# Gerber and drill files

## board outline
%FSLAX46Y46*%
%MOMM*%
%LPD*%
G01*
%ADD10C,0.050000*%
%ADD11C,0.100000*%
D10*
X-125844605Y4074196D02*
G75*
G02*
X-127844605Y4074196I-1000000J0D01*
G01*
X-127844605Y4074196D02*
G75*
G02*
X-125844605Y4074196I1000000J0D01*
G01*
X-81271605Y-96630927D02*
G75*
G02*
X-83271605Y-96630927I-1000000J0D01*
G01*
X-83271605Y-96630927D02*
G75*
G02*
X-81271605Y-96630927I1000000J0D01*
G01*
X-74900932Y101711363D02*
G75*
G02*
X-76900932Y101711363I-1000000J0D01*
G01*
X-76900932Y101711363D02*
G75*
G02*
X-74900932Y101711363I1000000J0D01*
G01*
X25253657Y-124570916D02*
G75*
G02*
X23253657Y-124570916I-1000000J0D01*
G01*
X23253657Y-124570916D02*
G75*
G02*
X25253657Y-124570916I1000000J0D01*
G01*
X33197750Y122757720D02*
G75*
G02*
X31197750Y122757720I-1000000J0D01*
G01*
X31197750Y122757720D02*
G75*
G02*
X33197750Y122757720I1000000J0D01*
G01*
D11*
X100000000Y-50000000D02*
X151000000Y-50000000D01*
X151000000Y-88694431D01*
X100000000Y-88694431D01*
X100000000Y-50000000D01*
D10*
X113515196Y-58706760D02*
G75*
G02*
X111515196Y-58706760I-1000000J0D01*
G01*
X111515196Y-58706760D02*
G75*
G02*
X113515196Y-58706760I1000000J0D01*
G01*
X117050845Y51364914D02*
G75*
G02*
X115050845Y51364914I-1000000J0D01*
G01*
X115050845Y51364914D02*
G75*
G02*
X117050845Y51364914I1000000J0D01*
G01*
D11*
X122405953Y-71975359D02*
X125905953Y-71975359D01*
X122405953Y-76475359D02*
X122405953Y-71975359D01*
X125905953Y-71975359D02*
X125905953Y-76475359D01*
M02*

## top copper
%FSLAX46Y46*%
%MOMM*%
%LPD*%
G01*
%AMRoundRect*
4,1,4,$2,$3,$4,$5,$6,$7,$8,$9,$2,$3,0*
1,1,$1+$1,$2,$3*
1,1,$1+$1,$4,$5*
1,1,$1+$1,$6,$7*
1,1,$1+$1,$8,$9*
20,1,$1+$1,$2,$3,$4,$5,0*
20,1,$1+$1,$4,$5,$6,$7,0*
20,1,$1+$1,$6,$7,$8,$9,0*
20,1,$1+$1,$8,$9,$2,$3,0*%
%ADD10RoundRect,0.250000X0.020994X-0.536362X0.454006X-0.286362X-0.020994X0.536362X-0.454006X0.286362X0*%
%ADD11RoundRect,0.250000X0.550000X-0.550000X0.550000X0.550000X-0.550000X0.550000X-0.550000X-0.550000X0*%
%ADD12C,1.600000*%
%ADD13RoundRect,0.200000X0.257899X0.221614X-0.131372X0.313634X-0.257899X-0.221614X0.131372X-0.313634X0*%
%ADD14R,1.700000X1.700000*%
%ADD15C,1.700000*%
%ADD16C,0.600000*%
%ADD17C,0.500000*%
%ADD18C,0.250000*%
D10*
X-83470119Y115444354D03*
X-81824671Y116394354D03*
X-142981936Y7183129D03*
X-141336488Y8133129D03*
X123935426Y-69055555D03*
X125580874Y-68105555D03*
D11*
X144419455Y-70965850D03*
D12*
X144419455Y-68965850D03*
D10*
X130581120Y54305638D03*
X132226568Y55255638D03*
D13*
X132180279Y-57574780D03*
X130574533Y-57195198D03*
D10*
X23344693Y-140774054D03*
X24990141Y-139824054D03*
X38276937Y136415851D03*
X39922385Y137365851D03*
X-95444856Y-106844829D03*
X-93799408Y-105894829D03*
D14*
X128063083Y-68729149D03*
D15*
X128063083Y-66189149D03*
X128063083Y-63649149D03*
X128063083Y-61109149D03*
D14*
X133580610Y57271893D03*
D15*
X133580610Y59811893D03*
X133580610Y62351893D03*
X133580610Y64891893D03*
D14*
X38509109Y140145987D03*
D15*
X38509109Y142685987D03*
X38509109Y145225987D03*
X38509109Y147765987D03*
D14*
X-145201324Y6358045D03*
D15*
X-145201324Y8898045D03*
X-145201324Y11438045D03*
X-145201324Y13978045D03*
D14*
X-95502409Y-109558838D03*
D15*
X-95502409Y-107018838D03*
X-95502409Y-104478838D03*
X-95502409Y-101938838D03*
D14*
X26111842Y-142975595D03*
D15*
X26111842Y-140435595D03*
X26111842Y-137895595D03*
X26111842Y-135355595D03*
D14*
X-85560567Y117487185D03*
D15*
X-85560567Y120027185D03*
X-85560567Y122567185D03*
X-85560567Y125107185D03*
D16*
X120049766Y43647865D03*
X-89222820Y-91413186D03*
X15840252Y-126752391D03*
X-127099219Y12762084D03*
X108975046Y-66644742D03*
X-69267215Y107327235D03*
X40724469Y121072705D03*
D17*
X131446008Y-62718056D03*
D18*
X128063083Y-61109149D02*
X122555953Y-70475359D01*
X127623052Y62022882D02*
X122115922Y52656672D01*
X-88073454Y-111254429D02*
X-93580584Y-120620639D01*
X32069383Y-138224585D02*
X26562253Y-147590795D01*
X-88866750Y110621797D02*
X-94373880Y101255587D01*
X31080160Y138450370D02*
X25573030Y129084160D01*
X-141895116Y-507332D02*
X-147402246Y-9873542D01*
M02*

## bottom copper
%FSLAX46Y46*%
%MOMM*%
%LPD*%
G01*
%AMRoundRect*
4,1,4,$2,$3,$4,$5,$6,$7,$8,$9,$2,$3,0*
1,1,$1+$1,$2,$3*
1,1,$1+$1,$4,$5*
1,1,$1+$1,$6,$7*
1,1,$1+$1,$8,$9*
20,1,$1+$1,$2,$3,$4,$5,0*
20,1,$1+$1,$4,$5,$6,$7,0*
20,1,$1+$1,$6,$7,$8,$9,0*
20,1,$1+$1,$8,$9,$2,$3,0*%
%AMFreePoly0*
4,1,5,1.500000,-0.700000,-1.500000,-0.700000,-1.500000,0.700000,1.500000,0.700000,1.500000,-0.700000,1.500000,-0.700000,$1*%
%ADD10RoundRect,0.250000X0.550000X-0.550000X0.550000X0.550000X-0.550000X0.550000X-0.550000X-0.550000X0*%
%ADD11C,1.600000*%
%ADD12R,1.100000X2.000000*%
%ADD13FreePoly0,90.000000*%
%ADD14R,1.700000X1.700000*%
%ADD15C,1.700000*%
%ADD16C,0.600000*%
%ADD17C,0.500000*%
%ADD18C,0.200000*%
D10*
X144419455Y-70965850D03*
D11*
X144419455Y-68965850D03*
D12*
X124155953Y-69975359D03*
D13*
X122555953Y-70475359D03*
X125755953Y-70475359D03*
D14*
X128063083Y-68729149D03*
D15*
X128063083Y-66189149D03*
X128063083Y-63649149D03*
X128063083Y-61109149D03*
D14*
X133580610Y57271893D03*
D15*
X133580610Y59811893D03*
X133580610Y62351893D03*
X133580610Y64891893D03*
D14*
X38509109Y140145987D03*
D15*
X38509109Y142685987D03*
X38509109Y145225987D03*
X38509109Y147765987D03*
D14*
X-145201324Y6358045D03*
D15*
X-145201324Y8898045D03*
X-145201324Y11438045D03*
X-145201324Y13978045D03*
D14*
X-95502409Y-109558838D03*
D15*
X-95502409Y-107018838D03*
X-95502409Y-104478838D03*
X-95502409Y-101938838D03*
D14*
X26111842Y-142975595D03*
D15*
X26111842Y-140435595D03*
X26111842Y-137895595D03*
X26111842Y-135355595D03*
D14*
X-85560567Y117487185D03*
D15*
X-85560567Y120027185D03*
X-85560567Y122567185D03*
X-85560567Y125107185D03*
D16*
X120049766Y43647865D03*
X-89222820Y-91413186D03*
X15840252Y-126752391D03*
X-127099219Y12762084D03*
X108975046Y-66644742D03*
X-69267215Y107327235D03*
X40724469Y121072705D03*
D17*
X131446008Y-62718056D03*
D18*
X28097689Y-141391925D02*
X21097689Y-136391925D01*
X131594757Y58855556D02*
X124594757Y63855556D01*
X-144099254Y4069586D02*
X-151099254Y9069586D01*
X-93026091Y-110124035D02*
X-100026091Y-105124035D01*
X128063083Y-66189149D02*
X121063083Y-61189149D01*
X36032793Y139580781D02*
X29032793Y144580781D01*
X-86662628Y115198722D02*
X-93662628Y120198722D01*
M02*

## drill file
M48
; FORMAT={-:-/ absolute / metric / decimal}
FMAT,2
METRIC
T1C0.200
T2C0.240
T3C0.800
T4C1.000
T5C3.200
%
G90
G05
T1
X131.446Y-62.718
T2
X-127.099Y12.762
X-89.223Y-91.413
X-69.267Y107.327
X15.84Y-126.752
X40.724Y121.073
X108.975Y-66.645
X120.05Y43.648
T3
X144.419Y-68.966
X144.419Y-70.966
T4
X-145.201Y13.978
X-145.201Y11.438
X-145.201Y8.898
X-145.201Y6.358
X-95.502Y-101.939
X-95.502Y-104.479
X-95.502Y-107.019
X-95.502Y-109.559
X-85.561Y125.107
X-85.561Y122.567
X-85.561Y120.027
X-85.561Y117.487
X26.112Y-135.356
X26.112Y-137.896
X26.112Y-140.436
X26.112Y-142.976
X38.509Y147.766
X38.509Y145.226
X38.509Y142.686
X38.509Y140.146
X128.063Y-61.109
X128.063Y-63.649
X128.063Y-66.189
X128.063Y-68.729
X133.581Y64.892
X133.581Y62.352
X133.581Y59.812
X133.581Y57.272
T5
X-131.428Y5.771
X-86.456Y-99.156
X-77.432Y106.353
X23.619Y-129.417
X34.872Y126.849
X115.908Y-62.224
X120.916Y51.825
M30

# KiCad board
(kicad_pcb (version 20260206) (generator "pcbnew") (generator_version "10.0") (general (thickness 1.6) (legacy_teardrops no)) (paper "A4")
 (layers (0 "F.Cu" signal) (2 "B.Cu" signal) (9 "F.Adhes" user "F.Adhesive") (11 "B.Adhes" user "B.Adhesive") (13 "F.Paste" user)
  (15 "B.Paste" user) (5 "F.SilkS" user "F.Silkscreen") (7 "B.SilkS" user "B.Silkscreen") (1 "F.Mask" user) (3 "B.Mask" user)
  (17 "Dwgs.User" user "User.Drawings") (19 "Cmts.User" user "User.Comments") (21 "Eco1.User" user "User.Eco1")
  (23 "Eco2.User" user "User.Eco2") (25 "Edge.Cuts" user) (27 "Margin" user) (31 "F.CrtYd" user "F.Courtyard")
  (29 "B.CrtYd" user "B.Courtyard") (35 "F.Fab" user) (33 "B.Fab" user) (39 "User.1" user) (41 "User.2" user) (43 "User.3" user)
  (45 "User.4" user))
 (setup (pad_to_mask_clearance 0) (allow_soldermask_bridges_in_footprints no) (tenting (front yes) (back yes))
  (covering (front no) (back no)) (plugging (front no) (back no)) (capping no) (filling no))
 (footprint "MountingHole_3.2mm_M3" (layer "F.Cu") (at -77.432084 -106.352638 45)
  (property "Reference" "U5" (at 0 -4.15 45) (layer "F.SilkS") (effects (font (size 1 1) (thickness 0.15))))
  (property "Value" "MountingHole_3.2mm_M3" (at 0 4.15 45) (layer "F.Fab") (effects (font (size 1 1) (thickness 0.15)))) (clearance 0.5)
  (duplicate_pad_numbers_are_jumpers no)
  (pad "" np_thru_hole circle (at 0 0 45) (size 3.2 3.2) (drill 3.2) (layers "*.Cu" "*.Mask")))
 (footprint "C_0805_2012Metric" (layer "F.Cu") (at -82.647395 -115.919354 30)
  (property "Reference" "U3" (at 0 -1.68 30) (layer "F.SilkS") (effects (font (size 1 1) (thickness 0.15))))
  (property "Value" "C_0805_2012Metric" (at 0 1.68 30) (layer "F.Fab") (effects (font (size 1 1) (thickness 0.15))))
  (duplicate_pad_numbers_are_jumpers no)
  (pad "1" smd roundrect (at -0.95 0 30) (size 1 1.45) (layers "F.Cu" "F.Mask" "F.Paste") (roundrect_rratio 0.25) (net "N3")
   (clearance 0.35))
  (pad "2" smd roundrect (at 0.95 0 30) (size 1 1.45) (layers "F.Cu" "F.Mask" "F.Paste") (roundrect_rratio 0.25)))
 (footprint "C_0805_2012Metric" (layer "F.Cu") (at -142.159212 -7.658129 30)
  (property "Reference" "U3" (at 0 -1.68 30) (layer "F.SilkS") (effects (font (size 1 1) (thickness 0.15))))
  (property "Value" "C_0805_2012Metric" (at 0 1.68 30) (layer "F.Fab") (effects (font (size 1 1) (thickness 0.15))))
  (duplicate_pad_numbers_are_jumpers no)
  (pad "1" smd roundrect (at -0.95 0 30) (size 1 1.45) (layers "F.Cu" "F.Mask" "F.Paste") (roundrect_rratio 0.25) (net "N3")
   (clearance 0.35))
  (pad "2" smd roundrect (at 0.95 0 30) (size 1 1.45) (layers "F.Cu" "F.Mask" "F.Paste") (roundrect_rratio 0.25)))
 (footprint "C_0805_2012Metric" (layer "F.Cu") (at 124.75815 68.580555 30)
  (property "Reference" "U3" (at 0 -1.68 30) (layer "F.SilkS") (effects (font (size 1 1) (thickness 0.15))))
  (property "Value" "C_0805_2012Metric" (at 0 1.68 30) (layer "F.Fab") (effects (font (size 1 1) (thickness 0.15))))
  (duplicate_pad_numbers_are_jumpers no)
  (pad "1" smd roundrect (at -0.95 0 30) (size 1 1.45) (layers "F.Cu" "F.Mask" "F.Paste") (roundrect_rratio 0.25) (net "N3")
   (clearance 0.35))
  (pad "2" smd roundrect (at 0.95 0 30) (size 1 1.45) (layers "F.Cu" "F.Mask" "F.Paste") (roundrect_rratio 0.25)))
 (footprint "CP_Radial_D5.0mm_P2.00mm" (layer "F.Cu") (at 144.419455 70.96585 90)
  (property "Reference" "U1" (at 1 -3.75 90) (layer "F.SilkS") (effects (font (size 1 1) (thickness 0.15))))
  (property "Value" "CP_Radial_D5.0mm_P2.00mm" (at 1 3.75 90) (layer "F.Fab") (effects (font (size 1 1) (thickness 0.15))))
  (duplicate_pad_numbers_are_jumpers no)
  (pad "1" thru_hole roundrect (at 0 0 90) (size 1.6 1.6) (drill 0.8) (layers "*.Cu" "*.Mask") (remove_unused_layers no)
   (roundrect_rratio 0.15625) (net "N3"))
  (pad "2" thru_hole circle (at 2 0 90) (size 1.6 1.6) (drill 0.8) (layers "*.Cu" "*.Mask") (remove_unused_layers no) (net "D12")))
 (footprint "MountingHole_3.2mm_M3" (layer "F.Cu") (at 120.916466 -51.824891 45)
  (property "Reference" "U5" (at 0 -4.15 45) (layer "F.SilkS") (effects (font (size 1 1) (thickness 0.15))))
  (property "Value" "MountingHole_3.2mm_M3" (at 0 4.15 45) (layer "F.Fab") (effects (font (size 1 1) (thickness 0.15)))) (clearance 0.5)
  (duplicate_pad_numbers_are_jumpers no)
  (pad "" np_thru_hole circle (at 0 0 45) (size 3.2 3.2) (drill 3.2) (layers "*.Cu" "*.Mask")))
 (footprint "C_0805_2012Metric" (layer "F.Cu") (at 131.403844 -54.780638 30)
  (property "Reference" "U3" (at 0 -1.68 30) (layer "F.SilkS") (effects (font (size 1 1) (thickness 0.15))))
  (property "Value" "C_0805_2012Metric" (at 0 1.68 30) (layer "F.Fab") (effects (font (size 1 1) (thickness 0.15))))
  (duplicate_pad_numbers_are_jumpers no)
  (pad "1" smd roundrect (at -0.95 0 30) (size 1 1.45) (layers "F.Cu" "F.Mask" "F.Paste") (roundrect_rratio 0.25) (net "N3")
   (clearance 0.35))
  (pad "2" smd roundrect (at 0.95 0 30) (size 1 1.45) (layers "F.Cu" "F.Mask" "F.Paste") (roundrect_rratio 0.25)))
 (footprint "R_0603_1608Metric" (layer "F.Cu") (at 131.377406 57.384989 166.7)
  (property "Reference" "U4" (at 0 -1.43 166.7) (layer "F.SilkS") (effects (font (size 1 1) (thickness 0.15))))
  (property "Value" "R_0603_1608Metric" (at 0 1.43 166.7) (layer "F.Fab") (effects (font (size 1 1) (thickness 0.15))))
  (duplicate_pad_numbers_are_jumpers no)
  (pad "1" smd roundrect (at -0.825 0 166.7) (size 0.8 0.95) (layers "F.Cu" "F.Mask" "F.Paste") (roundrect_rratio 0.25) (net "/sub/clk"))
  (pad "2" smd roundrect (at 0.825 0 166.7) (size 0.8 0.95) (layers "F.Cu" "F.Mask" "F.Paste") (roundrect_rratio 0.25) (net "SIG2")))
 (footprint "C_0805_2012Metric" (layer "F.Cu") (at 24.167417 140.299054 30)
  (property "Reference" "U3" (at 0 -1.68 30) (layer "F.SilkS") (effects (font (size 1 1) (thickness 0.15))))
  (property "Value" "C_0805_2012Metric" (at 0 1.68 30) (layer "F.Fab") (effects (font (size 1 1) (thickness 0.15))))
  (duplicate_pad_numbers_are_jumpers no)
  (pad "1" smd roundrect (at -0.95 0 30) (size 1 1.45) (layers "F.Cu" "F.Mask" "F.Paste") (roundrect_rratio 0.25) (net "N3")
   (clearance 0.35))
  (pad "2" smd roundrect (at 0.95 0 30) (size 1 1.45) (layers "F.Cu" "F.Mask" "F.Paste") (roundrect_rratio 0.25)))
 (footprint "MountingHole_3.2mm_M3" (layer "F.Cu") (at -131.427958 -5.770879 45)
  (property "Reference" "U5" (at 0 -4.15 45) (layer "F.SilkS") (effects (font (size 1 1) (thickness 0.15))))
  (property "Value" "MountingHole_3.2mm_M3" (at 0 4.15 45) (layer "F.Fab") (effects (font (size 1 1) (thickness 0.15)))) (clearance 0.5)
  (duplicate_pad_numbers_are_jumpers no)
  (pad "" np_thru_hole circle (at 0 0 45) (size 3.2 3.2) (drill 3.2) (layers "*.Cu" "*.Mask")))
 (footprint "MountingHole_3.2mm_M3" (layer "F.Cu") (at 34.871789 -126.848609 45)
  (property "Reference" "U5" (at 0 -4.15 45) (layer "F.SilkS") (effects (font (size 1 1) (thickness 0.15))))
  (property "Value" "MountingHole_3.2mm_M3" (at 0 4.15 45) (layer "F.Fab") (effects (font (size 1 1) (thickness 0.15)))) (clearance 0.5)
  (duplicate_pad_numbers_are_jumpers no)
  (pad "" np_thru_hole circle (at 0 0 45) (size 3.2 3.2) (drill 3.2) (layers "*.Cu" "*.Mask")))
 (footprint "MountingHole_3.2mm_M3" (layer "F.Cu") (at 115.908484 62.224067 45)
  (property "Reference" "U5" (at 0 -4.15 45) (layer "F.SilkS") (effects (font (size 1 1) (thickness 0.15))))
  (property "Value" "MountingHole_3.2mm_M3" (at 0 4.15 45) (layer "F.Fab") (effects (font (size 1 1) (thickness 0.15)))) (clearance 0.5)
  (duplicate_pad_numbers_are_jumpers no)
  (pad "" np_thru_hole circle (at 0 0 45) (size 3.2 3.2) (drill 3.2) (layers "*.Cu" "*.Mask")))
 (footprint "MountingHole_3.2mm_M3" (layer "F.Cu") (at 23.61941 129.416902 45)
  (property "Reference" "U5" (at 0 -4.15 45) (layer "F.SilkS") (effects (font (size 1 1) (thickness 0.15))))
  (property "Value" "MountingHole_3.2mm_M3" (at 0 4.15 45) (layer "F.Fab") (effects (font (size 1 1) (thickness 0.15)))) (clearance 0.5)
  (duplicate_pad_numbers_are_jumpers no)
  (pad "" np_thru_hole circle (at 0 0 45) (size 3.2 3.2) (drill 3.2) (layers "*.Cu" "*.Mask")))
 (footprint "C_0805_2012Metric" (layer "F.Cu") (at 39.099661 -136.890851 30)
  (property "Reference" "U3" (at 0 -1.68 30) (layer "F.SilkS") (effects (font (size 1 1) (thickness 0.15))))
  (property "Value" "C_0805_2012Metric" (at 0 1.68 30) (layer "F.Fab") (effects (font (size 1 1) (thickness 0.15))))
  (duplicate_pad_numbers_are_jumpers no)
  (pad "1" smd roundrect (at -0.95 0 30) (size 1 1.45) (layers "F.Cu" "F.Mask" "F.Paste") (roundrect_rratio 0.25) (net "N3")
   (clearance 0.35))
  (pad "2" smd roundrect (at 0.95 0 30) (size 1 1.45) (layers "F.Cu" "F.Mask" "F.Paste") (roundrect_rratio 0.25)))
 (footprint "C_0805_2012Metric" (layer "F.Cu") (at -94.622132 106.369829 30)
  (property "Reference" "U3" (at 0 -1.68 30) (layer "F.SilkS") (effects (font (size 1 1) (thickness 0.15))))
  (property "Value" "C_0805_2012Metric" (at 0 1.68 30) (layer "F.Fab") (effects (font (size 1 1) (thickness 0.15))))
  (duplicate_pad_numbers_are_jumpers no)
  (pad "1" smd roundrect (at -0.95 0 30) (size 1 1.45) (layers "F.Cu" "F.Mask" "F.Paste") (roundrect_rratio 0.25) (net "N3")
   (clearance 0.35))
  (pad "2" smd roundrect (at 0.95 0 30) (size 1 1.45) (layers "F.Cu" "F.Mask" "F.Paste") (roundrect_rratio 0.25)))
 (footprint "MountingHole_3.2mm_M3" (layer "F.Cu") (at -86.455797 99.156474 45)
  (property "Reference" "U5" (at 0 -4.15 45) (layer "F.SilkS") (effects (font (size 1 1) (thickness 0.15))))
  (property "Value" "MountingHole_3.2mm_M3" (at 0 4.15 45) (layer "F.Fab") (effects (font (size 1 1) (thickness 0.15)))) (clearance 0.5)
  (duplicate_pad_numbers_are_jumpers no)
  (pad "" np_thru_hole circle (at 0 0 45) (size 3.2 3.2) (drill 3.2) (layers "*.Cu" "*.Mask")))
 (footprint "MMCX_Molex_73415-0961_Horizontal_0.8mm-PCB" (layer "B.Cu") (at 124.155953 72.725359 90)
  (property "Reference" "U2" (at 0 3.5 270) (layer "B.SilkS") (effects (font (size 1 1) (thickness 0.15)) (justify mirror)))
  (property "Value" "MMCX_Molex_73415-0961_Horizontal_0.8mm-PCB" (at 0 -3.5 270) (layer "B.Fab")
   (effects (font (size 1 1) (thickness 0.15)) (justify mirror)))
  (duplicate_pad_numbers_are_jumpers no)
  (fp_line (start 0.75 -1.75) (end 0.75 1.75) (stroke (width 0.1) (type solid)) (layer "Edge.Cuts"))
  (fp_line (start -3.75 -1.75) (end 0.75 -1.75) (stroke (width 0.1) (type solid)) (layer "Edge.Cuts"))
  (fp_line (start 0.75 1.75) (end -3.75 1.75) (stroke (width 0.1) (type solid)) (layer "Edge.Cuts"))
  (pad "1" smd rect (at 2.75 0 90) (size 2 1.1) (layers "B.Cu" "B.Mask" "B.Paste") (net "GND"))
  (pad "2" smd custom (at 2.25 -1.6 90) (size 3 1.4) (layers "B.Cu" "B.Mask" "B.Paste") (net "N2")
   (options (clearance outline) (anchor rect)) (primitives))
  (pad "2" smd custom (at 2.25 1.6 90) (size 3 1.4) (layers "B.Cu" "B.Mask" "B.Paste") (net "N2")
   (options (clearance outline) (anchor rect)) (primitives)))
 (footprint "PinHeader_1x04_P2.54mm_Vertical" (layer "B.Cu") (at 128.063083 68.729149)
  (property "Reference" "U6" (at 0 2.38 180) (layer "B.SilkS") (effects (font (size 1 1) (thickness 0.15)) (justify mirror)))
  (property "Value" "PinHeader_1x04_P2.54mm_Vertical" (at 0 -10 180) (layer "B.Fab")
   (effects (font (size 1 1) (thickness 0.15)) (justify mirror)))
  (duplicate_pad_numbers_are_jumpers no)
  (pad "1" thru_hole rect (at 0 0) (size 1.7 1.7) (drill 1) (layers "*.Cu" "*.Mask") (remove_unused_layers no) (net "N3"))
  (pad "2" thru_hole circle (at 0 -2.54) (size 1.7 1.7) (drill 1) (layers "*.Cu" "*.Mask") (remove_unused_layers no) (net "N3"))
  (pad "3" thru_hole circle (at 0 -5.08) (size 1.7 1.7) (drill 1) (layers "*.Cu" "*.Mask") (remove_unused_layers no) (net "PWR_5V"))
  (pad "4" thru_hole circle (at 0 -7.62) (size 1.7 1.7) (drill 1) (layers "*.Cu" "*.Mask") (remove_unused_layers no)))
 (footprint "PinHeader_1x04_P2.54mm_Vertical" (layer "B.Cu") (at 133.58061 -57.271893)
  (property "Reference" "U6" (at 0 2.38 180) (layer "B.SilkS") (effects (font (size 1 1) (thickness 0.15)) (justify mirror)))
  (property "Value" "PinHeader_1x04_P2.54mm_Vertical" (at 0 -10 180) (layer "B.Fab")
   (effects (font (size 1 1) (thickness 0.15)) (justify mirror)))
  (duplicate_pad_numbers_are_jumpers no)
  (pad "1" thru_hole rect (at 0 0) (size 1.7 1.7) (drill 1) (layers "*.Cu" "*.Mask") (remove_unused_layers no) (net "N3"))
  (pad "2" thru_hole circle (at 0 -2.54) (size 1.7 1.7) (drill 1) (layers "*.Cu" "*.Mask") (remove_unused_layers no) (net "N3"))
  (pad "3" thru_hole circle (at 0 -5.08) (size 1.7 1.7) (drill 1) (layers "*.Cu" "*.Mask") (remove_unused_layers no) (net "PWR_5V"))
  (pad "4" thru_hole circle (at 0 -7.62) (size 1.7 1.7) (drill 1) (layers "*.Cu" "*.Mask") (remove_unused_layers no)))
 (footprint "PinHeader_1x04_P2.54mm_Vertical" (layer "B.Cu") (at 38.509109 -140.145987)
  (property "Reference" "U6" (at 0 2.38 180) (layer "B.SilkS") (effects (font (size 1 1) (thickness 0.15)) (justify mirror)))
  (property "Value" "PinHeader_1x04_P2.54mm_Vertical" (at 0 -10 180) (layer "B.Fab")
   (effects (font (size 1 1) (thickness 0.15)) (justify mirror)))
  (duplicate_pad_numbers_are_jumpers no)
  (pad "1" thru_hole rect (at 0 0) (size 1.7 1.7) (drill 1) (layers "*.Cu" "*.Mask") (remove_unused_layers no) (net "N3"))
  (pad "2" thru_hole circle (at 0 -2.54) (size 1.7 1.7) (drill 1) (layers "*.Cu" "*.Mask") (remove_unused_layers no) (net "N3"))
  (pad "3" thru_hole circle (at 0 -5.08) (size 1.7 1.7) (drill 1) (layers "*.Cu" "*.Mask") (remove_unused_layers no) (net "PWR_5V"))
  (pad "4" thru_hole circle (at 0 -7.62) (size 1.7 1.7) (drill 1) (layers "*.Cu" "*.Mask") (remove_unused_layers no)))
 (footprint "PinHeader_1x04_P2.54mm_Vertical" (layer "B.Cu") (at -145.201324 -6.358045)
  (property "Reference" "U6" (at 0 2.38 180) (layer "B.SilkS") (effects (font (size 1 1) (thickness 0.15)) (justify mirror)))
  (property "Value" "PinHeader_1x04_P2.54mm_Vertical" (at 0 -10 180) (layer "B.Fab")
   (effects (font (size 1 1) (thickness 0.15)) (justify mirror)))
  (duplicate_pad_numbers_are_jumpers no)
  (pad "1" thru_hole rect (at 0 0) (size 1.7 1.7) (drill 1) (layers "*.Cu" "*.Mask") (remove_unused_layers no) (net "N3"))
  (pad "2" thru_hole circle (at 0 -2.54) (size 1.7 1.7) (drill 1) (layers "*.Cu" "*.Mask") (remove_unused_layers no) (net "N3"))
  (pad "3" thru_hole circle (at 0 -5.08) (size 1.7 1.7) (drill 1) (layers "*.Cu" "*.Mask") (remove_unused_layers no) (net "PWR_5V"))
  (pad "4" thru_hole circle (at 0 -7.62) (size 1.7 1.7) (drill 1) (layers "*.Cu" "*.Mask") (remove_unused_layers no)))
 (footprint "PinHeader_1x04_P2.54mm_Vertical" (layer "B.Cu") (at -95.502409 109.558838)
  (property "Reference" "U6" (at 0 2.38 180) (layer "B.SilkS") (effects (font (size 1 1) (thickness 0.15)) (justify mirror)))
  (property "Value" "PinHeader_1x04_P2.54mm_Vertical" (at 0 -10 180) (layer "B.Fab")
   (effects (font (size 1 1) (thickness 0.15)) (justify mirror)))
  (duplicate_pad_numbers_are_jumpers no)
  (pad "1" thru_hole rect (at 0 0) (size 1.7 1.7) (drill 1) (layers "*.Cu" "*.Mask") (remove_unused_layers no) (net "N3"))
  (pad "2" thru_hole circle (at 0 -2.54) (size 1.7 1.7) (drill 1) (layers "*.Cu" "*.Mask") (remove_unused_layers no) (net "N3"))
  (pad "3" thru_hole circle (at 0 -5.08) (size 1.7 1.7) (drill 1) (layers "*.Cu" "*.Mask") (remove_unused_layers no) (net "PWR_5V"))
  (pad "4" thru_hole circle (at 0 -7.62) (size 1.7 1.7) (drill 1) (layers "*.Cu" "*.Mask") (remove_unused_layers no)))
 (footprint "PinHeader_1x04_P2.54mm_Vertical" (layer "B.Cu") (at 26.111842 142.975595)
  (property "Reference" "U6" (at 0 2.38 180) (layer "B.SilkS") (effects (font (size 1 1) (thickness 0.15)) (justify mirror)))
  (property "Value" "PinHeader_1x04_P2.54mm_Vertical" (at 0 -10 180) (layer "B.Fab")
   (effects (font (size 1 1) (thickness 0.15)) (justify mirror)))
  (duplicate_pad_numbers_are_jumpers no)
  (pad "1" thru_hole rect (at 0 0) (size 1.7 1.7) (drill 1) (layers "*.Cu" "*.Mask") (remove_unused_layers no) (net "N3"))
  (pad "2" thru_hole circle (at 0 -2.54) (size 1.7 1.7) (drill 1) (layers "*.Cu" "*.Mask") (remove_unused_layers no) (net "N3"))
  (pad "3" thru_hole circle (at 0 -5.08) (size 1.7 1.7) (drill 1) (layers "*.Cu" "*.Mask") (remove_unused_layers no) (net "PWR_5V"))
  (pad "4" thru_hole circle (at 0 -7.62) (size 1.7 1.7) (drill 1) (layers "*.Cu" "*.Mask") (remove_unused_layers no)))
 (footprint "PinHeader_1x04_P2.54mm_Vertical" (layer "B.Cu") (at -85.560567 -117.487185)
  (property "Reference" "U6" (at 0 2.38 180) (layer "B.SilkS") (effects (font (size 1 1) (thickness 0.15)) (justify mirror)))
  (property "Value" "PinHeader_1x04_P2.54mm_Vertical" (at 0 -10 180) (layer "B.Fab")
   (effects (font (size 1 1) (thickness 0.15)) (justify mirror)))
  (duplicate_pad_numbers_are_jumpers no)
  (pad "1" thru_hole rect (at 0 0) (size 1.7 1.7) (drill 1) (layers "*.Cu" "*.Mask") (remove_unused_layers no) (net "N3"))
  (pad "2" thru_hole circle (at 0 -2.54) (size 1.7 1.7) (drill 1) (layers "*.Cu" "*.Mask") (remove_unused_layers no) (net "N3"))
  (pad "3" thru_hole circle (at 0 -5.08) (size 1.7 1.7) (drill 1) (layers "*.Cu" "*.Mask") (remove_unused_layers no) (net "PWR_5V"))
  (pad "4" thru_hole circle (at 0 -7.62) (size 1.7 1.7) (drill 1) (layers "*.Cu" "*.Mask") (remove_unused_layers no)))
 (gr_circle (center -126.844605 -4.074196) (end -125.844605 -4.074196) (stroke (width 0.05) (type default)) (fill no) (layer "Edge.Cuts"))
 (gr_circle (center -82.271605 96.630927) (end -81.271605 96.630927) (stroke (width 0.05) (type default)) (fill no) (layer "Edge.Cuts"))
 (gr_circle (center -75.900932 -101.711363) (end -74.900932 -101.711363) (stroke (width 0.05) (type default)) (fill no) (layer "Edge.Cuts"))
 (gr_circle (center 24.253657 124.570916) (end 25.253657 124.570916) (stroke (width 0.05) (type default)) (fill no) (layer "Edge.Cuts"))
 (gr_circle (center 32.19775 -122.75772) (end 33.19775 -122.75772) (stroke (width 0.05) (type default)) (fill no) (layer "Edge.Cuts"))
 (gr_rect (start 100 50) (end 151 88.694431) (stroke (width 0.1) (type default)) (fill no) (layer "Edge.Cuts"))
 (gr_circle (center 112.515196 58.70676) (end 113.515196 58.70676) (stroke (width 0.05) (type default)) (fill no) (layer "Edge.Cuts"))
 (gr_circle (center 116.050845 -51.364914) (end 117.050845 -51.364914) (stroke (width 0.05) (type default)) (fill no) (layer "Edge.Cuts"))
 (segment (start 128.063083 61.109149) (end 122.555953 70.475359) (width 0.25) (layer "F.Cu") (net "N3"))
 (segment (start 127.623052 -62.022882) (end 122.115922 -52.656672) (width 0.25) (layer "F.Cu") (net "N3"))
 (segment (start -88.073454 111.254429) (end -93.580584 120.620639) (width 0.25) (layer "F.Cu") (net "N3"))
 (segment (start 32.069383 138.224585) (end 26.562253 147.590795) (width 0.25) (layer "F.Cu") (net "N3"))
 (segment (start -88.86675 -110.621797) (end -94.37388 -101.255587) (width 0.25) (layer "F.Cu") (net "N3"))
 (segment (start 31.08016 -138.45037) (end 25.57303 -129.08416) (width 0.25) (layer "F.Cu") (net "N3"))
 (segment (start -141.895116 0.507332) (end -147.402246 9.873542) (width 0.25) (layer "F.Cu") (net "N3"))
 (segment (start 28.097689 141.391925) (end 21.097689 136.391925) (width 0.2) (layer "B.Cu") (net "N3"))
 (segment (start 131.594757 -58.855556) (end 124.594757 -63.855556) (width 0.2) (layer "B.Cu") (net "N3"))
 (segment (start -144.099254 -4.069586) (end -151.099254 -9.069586) (width 0.2) (layer "B.Cu") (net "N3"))
 (segment (start -93.026091 110.124035) (end -100.026091 105.124035) (width 0.2) (layer "B.Cu") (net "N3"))
 (segment (start 128.063083 66.189149) (end 121.063083 61.189149) (width 0.2) (layer "B.Cu") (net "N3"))
 (segment (start 36.032793 -139.580781) (end 29.032793 -144.580781) (width 0.2) (layer "B.Cu") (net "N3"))
 (segment (start -86.662628 -115.198722) (end -93.662628 -120.198722) (width 0.2) (layer "B.Cu") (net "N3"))
 (via (at 120.049766 -43.647865) (size 0.6) (drill 0.24) (layers "F.Cu" "B.Cu") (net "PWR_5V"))
 (via (at -89.22282 91.413186) (size 0.6) (drill 0.24) (layers "F.Cu" "B.Cu") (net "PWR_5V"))
 (via (at 15.840252 126.752391) (size 0.6) (drill 0.24) (layers "F.Cu" "B.Cu") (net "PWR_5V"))
 (via (at -127.099219 -12.762084) (size 0.6) (drill 0.24) (layers "F.Cu" "B.Cu") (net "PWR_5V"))
 (via (at 108.975046 66.644742) (size 0.6) (drill 0.24) (layers "F.Cu" "B.Cu") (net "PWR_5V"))
 (via (at -69.267215 -107.327235) (size 0.6) (drill 0.24) (layers "F.Cu" "B.Cu") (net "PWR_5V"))
 (via (at 40.724469 -121.072705) (size 0.6) (drill 0.24) (layers "F.Cu" "B.Cu") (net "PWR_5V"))
 (via (at 131.446008 62.718056) (size 0.5) (drill 0.2) (layers "F.Cu" "B.Cu") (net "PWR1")))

